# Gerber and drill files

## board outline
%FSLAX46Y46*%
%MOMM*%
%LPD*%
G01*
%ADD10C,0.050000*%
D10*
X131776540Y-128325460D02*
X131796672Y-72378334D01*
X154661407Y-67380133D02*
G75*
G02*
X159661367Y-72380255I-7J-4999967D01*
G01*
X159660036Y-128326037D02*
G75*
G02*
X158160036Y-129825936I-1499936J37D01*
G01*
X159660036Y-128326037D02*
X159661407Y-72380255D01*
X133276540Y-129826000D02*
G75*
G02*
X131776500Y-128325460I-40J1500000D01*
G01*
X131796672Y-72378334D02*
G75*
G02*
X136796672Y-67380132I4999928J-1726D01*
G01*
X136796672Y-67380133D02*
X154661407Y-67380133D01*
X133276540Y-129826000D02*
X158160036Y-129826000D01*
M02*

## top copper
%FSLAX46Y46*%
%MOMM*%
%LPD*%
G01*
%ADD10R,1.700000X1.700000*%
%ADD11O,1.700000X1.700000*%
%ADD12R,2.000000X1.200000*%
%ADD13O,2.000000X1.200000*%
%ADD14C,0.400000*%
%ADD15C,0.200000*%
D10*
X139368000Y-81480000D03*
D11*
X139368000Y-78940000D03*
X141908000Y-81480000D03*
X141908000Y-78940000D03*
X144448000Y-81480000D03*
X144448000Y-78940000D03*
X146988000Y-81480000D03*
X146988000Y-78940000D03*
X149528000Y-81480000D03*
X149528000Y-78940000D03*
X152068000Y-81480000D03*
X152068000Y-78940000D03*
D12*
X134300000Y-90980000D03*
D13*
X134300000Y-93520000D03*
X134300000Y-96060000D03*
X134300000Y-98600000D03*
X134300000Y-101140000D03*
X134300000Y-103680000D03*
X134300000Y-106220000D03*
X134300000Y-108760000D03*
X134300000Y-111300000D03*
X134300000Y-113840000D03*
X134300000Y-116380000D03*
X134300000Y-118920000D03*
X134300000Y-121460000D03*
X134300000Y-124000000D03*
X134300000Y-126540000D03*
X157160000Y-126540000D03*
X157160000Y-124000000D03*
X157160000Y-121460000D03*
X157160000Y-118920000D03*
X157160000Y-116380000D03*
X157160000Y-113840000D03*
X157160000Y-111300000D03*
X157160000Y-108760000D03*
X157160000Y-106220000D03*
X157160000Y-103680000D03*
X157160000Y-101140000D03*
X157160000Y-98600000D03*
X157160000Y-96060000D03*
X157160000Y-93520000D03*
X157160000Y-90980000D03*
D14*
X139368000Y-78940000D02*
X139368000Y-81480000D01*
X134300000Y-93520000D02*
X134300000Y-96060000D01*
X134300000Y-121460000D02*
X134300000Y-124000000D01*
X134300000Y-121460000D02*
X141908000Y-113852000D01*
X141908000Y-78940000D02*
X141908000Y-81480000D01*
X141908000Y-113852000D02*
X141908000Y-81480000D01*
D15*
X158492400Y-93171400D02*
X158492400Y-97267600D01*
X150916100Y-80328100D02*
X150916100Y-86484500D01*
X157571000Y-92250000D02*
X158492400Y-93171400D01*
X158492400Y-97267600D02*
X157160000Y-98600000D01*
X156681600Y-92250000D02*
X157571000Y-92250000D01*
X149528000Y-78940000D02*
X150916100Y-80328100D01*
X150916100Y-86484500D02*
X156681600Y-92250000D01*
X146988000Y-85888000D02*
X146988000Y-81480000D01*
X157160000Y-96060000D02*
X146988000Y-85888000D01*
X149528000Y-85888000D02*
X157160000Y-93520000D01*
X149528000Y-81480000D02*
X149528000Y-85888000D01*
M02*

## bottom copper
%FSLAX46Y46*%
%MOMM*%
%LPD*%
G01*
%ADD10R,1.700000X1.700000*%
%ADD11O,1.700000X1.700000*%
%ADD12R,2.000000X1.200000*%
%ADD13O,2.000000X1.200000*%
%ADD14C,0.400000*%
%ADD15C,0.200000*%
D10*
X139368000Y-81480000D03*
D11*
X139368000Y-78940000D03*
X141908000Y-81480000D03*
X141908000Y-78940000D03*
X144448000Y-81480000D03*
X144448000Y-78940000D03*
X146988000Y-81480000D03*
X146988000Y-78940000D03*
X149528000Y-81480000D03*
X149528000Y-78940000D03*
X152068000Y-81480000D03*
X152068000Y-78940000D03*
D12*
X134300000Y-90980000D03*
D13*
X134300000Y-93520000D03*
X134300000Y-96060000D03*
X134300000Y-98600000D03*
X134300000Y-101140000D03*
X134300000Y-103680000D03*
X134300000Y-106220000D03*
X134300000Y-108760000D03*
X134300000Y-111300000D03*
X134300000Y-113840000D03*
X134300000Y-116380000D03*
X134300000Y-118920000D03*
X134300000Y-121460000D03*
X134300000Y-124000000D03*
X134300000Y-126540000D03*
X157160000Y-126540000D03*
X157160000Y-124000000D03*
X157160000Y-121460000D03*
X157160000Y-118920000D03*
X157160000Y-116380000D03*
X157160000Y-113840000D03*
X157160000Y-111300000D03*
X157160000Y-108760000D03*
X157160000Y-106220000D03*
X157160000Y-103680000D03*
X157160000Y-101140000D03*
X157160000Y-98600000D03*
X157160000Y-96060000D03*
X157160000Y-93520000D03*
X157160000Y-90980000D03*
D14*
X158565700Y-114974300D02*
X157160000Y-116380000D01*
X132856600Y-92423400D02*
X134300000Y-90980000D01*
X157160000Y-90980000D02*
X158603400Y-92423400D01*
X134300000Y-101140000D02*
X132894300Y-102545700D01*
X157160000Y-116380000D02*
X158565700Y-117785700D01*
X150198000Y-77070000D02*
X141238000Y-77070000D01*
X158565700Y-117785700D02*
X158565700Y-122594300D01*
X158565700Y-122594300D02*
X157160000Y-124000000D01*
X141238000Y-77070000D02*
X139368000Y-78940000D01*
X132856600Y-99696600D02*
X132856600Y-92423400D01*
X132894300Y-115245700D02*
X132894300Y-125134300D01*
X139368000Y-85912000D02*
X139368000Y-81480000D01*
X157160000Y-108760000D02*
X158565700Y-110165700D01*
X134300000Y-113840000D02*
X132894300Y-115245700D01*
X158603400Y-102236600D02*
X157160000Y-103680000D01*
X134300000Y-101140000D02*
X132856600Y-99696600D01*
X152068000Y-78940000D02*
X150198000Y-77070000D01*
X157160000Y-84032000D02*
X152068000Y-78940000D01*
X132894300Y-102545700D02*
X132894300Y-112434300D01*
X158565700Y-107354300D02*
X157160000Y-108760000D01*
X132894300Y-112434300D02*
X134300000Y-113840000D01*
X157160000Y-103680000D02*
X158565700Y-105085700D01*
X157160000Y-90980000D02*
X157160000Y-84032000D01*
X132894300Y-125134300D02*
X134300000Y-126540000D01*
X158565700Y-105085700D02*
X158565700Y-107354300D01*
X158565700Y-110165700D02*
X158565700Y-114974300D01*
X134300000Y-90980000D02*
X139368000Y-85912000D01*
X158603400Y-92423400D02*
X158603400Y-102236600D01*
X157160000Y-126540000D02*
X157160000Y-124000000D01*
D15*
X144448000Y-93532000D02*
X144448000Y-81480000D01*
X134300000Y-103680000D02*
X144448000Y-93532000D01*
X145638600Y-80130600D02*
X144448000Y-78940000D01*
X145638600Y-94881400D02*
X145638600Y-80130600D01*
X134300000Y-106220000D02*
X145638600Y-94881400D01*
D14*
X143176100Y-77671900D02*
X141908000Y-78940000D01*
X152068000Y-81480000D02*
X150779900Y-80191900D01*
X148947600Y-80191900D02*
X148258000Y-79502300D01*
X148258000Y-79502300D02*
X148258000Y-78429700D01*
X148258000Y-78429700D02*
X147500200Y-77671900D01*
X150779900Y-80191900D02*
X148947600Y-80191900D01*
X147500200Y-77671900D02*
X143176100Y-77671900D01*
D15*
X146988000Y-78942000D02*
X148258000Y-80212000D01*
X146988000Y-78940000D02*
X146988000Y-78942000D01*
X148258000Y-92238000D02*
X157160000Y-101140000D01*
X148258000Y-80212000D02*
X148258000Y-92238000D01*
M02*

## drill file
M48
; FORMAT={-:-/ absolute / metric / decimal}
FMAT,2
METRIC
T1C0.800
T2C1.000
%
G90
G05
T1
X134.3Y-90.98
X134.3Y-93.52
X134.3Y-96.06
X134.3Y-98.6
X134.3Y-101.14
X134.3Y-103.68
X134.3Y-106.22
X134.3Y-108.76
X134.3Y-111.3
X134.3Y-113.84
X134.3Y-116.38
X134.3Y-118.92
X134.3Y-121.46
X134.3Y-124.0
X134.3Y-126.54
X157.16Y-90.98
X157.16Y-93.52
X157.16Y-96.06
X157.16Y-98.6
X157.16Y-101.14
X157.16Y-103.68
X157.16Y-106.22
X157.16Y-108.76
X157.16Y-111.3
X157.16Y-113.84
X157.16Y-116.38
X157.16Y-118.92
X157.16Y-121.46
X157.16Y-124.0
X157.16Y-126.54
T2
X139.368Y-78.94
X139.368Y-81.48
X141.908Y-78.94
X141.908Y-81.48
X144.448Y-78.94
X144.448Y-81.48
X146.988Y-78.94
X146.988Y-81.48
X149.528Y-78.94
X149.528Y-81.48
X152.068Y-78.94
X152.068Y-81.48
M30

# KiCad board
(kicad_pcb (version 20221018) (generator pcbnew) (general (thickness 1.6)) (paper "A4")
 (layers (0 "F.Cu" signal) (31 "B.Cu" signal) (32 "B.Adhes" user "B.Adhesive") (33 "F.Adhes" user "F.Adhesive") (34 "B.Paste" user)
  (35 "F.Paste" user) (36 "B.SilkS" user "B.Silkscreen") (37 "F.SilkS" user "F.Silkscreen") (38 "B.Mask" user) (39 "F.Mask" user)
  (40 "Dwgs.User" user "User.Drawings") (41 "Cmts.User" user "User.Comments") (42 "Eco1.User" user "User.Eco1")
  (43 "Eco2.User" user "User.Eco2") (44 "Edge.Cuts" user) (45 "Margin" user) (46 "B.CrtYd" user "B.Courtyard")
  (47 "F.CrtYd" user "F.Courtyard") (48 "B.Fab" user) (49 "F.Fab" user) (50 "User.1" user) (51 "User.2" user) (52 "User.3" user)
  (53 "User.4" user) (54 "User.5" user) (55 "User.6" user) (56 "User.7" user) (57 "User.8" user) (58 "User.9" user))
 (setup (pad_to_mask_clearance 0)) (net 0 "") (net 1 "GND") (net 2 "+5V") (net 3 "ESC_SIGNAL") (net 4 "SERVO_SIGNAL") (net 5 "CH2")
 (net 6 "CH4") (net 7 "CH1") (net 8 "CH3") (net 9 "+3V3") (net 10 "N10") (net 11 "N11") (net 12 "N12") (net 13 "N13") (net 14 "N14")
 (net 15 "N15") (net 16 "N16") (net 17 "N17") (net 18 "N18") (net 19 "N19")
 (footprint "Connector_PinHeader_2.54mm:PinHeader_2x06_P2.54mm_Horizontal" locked (layer "F.Cu") (at 139.368 81.48 90)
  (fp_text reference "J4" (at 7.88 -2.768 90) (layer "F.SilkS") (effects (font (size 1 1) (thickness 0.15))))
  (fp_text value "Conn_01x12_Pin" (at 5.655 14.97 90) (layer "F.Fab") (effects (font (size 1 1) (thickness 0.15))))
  (pad "1" thru_hole rect locked (at 0 0 90) (size 1.7 1.7) (drill 1) (layers "*.Cu" "*.Mask") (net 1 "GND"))
  (pad "2" thru_hole oval locked (at 2.54 0 90) (size 1.7 1.7) (drill 1) (layers "*.Cu" "*.Mask") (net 1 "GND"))
  (pad "3" thru_hole oval locked (at 0 2.54 90) (size 1.7 1.7) (drill 1) (layers "*.Cu" "*.Mask") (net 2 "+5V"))
  (pad "4" thru_hole oval locked (at 2.54 2.54 90) (size 1.7 1.7) (drill 1) (layers "*.Cu" "*.Mask") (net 2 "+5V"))
  (pad "5" thru_hole oval locked (at 0 5.08 90) (size 1.7 1.7) (drill 1) (layers "*.Cu" "*.Mask") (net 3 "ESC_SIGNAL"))
  (pad "6" thru_hole oval locked (at 2.54 5.08 90) (size 1.7 1.7) (drill 1) (layers "*.Cu" "*.Mask") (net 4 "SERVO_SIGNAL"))
  (pad "7" thru_hole oval locked (at 0 7.62 90) (size 1.7 1.7) (drill 1) (layers "*.Cu" "*.Mask") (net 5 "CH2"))
  (pad "8" thru_hole oval locked (at 2.54 7.62 90) (size 1.7 1.7) (drill 1) (layers "*.Cu" "*.Mask") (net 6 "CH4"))
  (pad "9" thru_hole oval locked (at 0 10.16 90) (size 1.7 1.7) (drill 1) (layers "*.Cu" "*.Mask") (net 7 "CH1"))
  (pad "10" thru_hole oval locked (at 2.54 10.16 90) (size 1.7 1.7) (drill 1) (layers "*.Cu" "*.Mask") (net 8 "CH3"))
  (pad "11" thru_hole oval locked (at 0 12.7 90) (size 1.7 1.7) (drill 1) (layers "*.Cu" "*.Mask") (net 2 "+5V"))
  (pad "12" thru_hole oval locked (at 2.54 12.7 90) (size 1.7 1.7) (drill 1) (layers "*.Cu" "*.Mask") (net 1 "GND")))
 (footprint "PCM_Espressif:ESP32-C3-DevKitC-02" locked (layer "F.Cu") (at 134.3 90.98)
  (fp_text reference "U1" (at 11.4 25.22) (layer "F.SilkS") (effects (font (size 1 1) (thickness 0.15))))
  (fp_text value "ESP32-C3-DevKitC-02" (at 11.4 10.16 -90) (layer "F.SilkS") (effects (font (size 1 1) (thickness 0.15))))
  (pad "1" thru_hole rect locked (at 0 0 270) (size 1.2 2) (drill 0.8) (layers "*.Cu" "*.Mask") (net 1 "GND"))
  (pad "2" thru_hole oval locked (at 0 2.54 270) (size 1.2 2) (drill 0.8) (layers "*.Cu" "*.Mask") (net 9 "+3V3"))
  (pad "3" thru_hole oval locked (at 0 5.08 270) (size 1.2 2) (drill 0.8) (layers "*.Cu" "*.Mask") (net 9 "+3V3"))
  (pad "4" thru_hole oval locked (at 0 7.62 270) (size 1.2 2) (drill 0.8) (layers "*.Cu" "*.Mask") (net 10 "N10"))
  (pad "5" thru_hole oval locked (at 0 10.16 270) (size 1.2 2) (drill 0.8) (layers "*.Cu" "*.Mask") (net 1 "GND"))
  (pad "6" thru_hole oval locked (at 0 12.7 270) (size 1.2 2) (drill 0.8) (layers "*.Cu" "*.Mask") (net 3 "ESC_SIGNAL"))
  (pad "7" thru_hole oval locked (at 0 15.24 270) (size 1.2 2) (drill 0.8) (layers "*.Cu" "*.Mask") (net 4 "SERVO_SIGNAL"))
  (pad "8" thru_hole oval locked (at 0 17.78 270) (size 1.2 2) (drill 0.8) (layers "*.Cu" "*.Mask") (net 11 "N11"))
  (pad "9" thru_hole oval locked (at 0 20.32 270) (size 1.2 2) (drill 0.8) (layers "*.Cu" "*.Mask") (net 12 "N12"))
  (pad "10" thru_hole oval locked (at 0 22.86 270) (size 1.2 2) (drill 0.8) (layers "*.Cu" "*.Mask") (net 1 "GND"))
  (pad "11" thru_hole oval locked (at 0 25.4 270) (size 1.2 2) (drill 0.8) (layers "*.Cu" "*.Mask") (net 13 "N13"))
  (pad "12" thru_hole oval locked (at 0 27.94 270) (size 1.2 2) (drill 0.8) (layers "*.Cu" "*.Mask") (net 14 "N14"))
  (pad "13" thru_hole oval locked (at 0 30.48 270) (size 1.2 2) (drill 0.8) (layers "*.Cu" "*.Mask") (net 2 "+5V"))
  (pad "14" thru_hole oval locked (at 0 33.02 270) (size 1.2 2) (drill 0.8) (layers "*.Cu" "*.Mask") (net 2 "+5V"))
  (pad "15" thru_hole oval locked (at 0 35.56 270) (size 1.2 2) (drill 0.8) (layers "*.Cu" "*.Mask") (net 1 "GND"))
  (pad "16" thru_hole oval locked (at 22.86 35.56 270) (size 1.2 2) (drill 0.8) (layers "*.Cu" "*.Mask") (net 1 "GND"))
  (pad "17" thru_hole oval locked (at 22.86 33.02 270) (size 1.2 2) (drill 0.8) (layers "*.Cu" "*.Mask") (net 1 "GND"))
  (pad "18" thru_hole oval locked (at 22.86 30.48 270) (size 1.2 2) (drill 0.8) (layers "*.Cu" "*.Mask") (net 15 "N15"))
  (pad "19" thru_hole oval locked (at 22.86 27.94 270) (size 1.2 2) (drill 0.8) (layers "*.Cu" "*.Mask") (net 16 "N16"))
  (pad "20" thru_hole oval locked (at 22.86 25.4 270) (size 1.2 2) (drill 0.8) (layers "*.Cu" "*.Mask") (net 1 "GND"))
  (pad "21" thru_hole oval locked (at 22.86 22.86 270) (size 1.2 2) (drill 0.8) (layers "*.Cu" "*.Mask") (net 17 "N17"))
  (pad "22" thru_hole oval locked (at 22.86 20.32 270) (size 1.2 2) (drill 0.8) (layers "*.Cu" "*.Mask") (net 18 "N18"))
  (pad "23" thru_hole oval locked (at 22.86 17.78 270) (size 1.2 2) (drill 0.8) (layers "*.Cu" "*.Mask") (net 1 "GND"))
  (pad "24" thru_hole oval locked (at 22.86 15.24 270) (size 1.2 2) (drill 0.8) (layers "*.Cu" "*.Mask") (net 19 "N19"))
  (pad "25" thru_hole oval locked (at 22.86 12.7 270) (size 1.2 2) (drill 0.8) (layers "*.Cu" "*.Mask") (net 1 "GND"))
  (pad "26" thru_hole oval locked (at 22.86 10.16 270) (size 1.2 2) (drill 0.8) (layers "*.Cu" "*.Mask") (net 6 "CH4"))
  (pad "27" thru_hole oval locked (at 22.86 7.62 270) (size 1.2 2) (drill 0.8) (layers "*.Cu" "*.Mask") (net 8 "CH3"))
  (pad "28" thru_hole oval locked (at 22.86 5.08 270) (size 1.2 2) (drill 0.8) (layers "*.Cu" "*.Mask") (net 5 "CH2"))
  (pad "29" thru_hole oval locked (at 22.86 2.54 270) (size 1.2 2) (drill 0.8) (layers "*.Cu" "*.Mask") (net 7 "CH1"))
  (pad "30" thru_hole oval locked (at 22.86 0 270) (size 1.2 2) (drill 0.8) (layers "*.Cu" "*.Mask") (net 1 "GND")))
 (gr_line (start 131.77654 128.32546) (end 131.796672 72.378334) (stroke (width 0.05) (type default)) (layer "Edge.Cuts"))
 (gr_arc (start 154.661407 67.380133) (mid 158.196984 68.844642) (end 159.661407 72.380255) (stroke (width 0.05) (type default))
  (layer "Edge.Cuts"))
 (gr_arc (start 159.660036 128.326037) (mid 159.220685 129.386686) (end 158.160036 129.826) (stroke (width 0.05) (type default))
  (layer "Edge.Cuts"))
 (gr_line (start 159.660036 128.326037) (end 159.661407 72.380255) (stroke (width 0.05) (type default)) (layer "Edge.Cuts"))
 (gr_arc (start 133.27654 129.826) (mid 132.215689 129.386469) (end 131.77654 128.32546) (stroke (width 0.05) (type default))
  (layer "Edge.Cuts"))
 (gr_arc (start 131.796672 72.378334) (mid 133.261761 68.843932) (end 136.796672 67.380133) (stroke (width 0.05) (type default))
  (layer "Edge.Cuts"))
 (gr_line (start 136.796672 67.380133) (end 154.661407 67.380133) (stroke (width 0.05) (type default)) (layer "Edge.Cuts"))
 (gr_line (start 133.27654 129.826) (end 158.160036 129.826) (stroke (width 0.05) (type default)) (layer "Edge.Cuts"))
 (segment (start 139.368 78.94) (end 139.368 81.48) (width 0.4) (layer "F.Cu") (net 1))
 (segment (start 158.5657 114.9743) (end 157.16 116.38) (width 0.4) (layer "B.Cu") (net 1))
 (segment (start 132.8566 92.4234) (end 134.3 90.98) (width 0.4) (layer "B.Cu") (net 1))
 (segment (start 157.16 90.98) (end 158.6034 92.4234) (width 0.4) (layer "B.Cu") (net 1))
 (segment (start 134.3 101.14) (end 132.8943 102.5457) (width 0.4) (layer "B.Cu") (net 1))
 (segment (start 157.16 116.38) (end 158.5657 117.7857) (width 0.4) (layer "B.Cu") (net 1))
 (segment (start 150.198 77.07) (end 141.238 77.07) (width 0.4) (layer "B.Cu") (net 1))
 (segment (start 158.5657 117.7857) (end 158.5657 122.5943) (width 0.4) (layer "B.Cu") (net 1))
 (segment (start 158.5657 122.5943) (end 157.16 124) (width 0.4) (layer "B.Cu") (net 1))
 (segment (start 141.238 77.07) (end 139.368 78.94) (width 0.4) (layer "B.Cu") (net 1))
 (segment (start 132.8566 99.6966) (end 132.8566 92.4234) (width 0.4) (layer "B.Cu") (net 1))
 (segment (start 132.8943 115.2457) (end 132.8943 125.1343) (width 0.4) (layer "B.Cu") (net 1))
 (segment (start 139.368 85.912) (end 139.368 81.48) (width 0.4) (layer "B.Cu") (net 1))
 (segment (start 157.16 108.76) (end 158.5657 110.1657) (width 0.4) (layer "B.Cu") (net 1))
 (segment (start 134.3 113.84) (end 132.8943 115.2457) (width 0.4) (layer "B.Cu") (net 1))
 (segment (start 158.6034 102.2366) (end 157.16 103.68) (width 0.4) (layer "B.Cu") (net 1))
 (segment (start 134.3 101.14) (end 132.8566 99.6966) (width 0.4) (layer "B.Cu") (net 1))
 (segment (start 152.068 78.94) (end 150.198 77.07) (width 0.4) (layer "B.Cu") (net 1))
 (segment (start 157.16 84.032) (end 152.068 78.94) (width 0.4) (layer "B.Cu") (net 1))
 (segment (start 132.8943 102.5457) (end 132.8943 112.4343) (width 0.4) (layer "B.Cu") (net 1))
 (segment (start 158.5657 107.3543) (end 157.16 108.76) (width 0.4) (layer "B.Cu") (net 1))
 (segment (start 132.8943 112.4343) (end 134.3 113.84) (width 0.4) (layer "B.Cu") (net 1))
 (segment (start 157.16 103.68) (end 158.5657 105.0857) (width 0.4) (layer "B.Cu") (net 1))
 (segment (start 157.16 90.98) (end 157.16 84.032) (width 0.4) (layer "B.Cu") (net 1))
 (segment (start 132.8943 125.1343) (end 134.3 126.54) (width 0.4) (layer "B.Cu") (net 1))
 (segment (start 158.5657 105.0857) (end 158.5657 107.3543) (width 0.4) (layer "B.Cu") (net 1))
 (segment (start 158.5657 110.1657) (end 158.5657 114.9743) (width 0.4) (layer "B.Cu") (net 1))
 (segment (start 134.3 90.98) (end 139.368 85.912) (width 0.4) (layer "B.Cu") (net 1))
 (segment (start 158.6034 92.4234) (end 158.6034 102.2366) (width 0.4) (layer "B.Cu") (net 1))
 (segment (start 157.16 126.54) (end 157.16 124) (width 0.4) (layer "B.Cu") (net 1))
 (segment (start 134.3 93.52) (end 134.3 96.06) (width 0.4) (layer "F.Cu") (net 9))
 (segment (start 144.448 93.532) (end 144.448 81.48) (width 0.2) (layer "B.Cu") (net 3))
 (segment (start 134.3 103.68) (end 144.448 93.532) (width 0.2) (layer "B.Cu") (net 3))
 (segment (start 145.6386 80.1306) (end 144.448 78.94) (width 0.2) (layer "B.Cu") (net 4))
 (segment (start 145.6386 94.8814) (end 145.6386 80.1306) (width 0.2) (layer "B.Cu") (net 4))
 (segment (start 134.3 106.22) (end 145.6386 94.8814) (width 0.2) (layer "B.Cu") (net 4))
 (segment (start 134.3 121.46) (end 134.3 124) (width 0.4) (layer "F.Cu") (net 2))
 (segment (start 134.3 121.46) (end 141.908 113.852) (width 0.4) (layer "F.Cu") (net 2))
 (segment (start 141.908 78.94) (end 141.908 81.48) (width 0.4) (layer "F.Cu") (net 2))
 (segment (start 141.908 113.852) (end 141.908 81.48) (width 0.4) (layer "F.Cu") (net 2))
 (segment (start 143.1761 77.6719) (end 141.908 78.94) (width 0.4) (layer "B.Cu") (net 2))
 (segment (start 152.068 81.48) (end 150.7799 80.1919) (width 0.4) (layer "B.Cu") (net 2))
 (segment (start 148.9476 80.1919) (end 148.258 79.5023) (width 0.4) (layer "B.Cu") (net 2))
 (segment (start 148.258 79.5023) (end 148.258 78.4297) (width 0.4) (layer "B.Cu") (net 2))
 (segment (start 148.258 78.4297) (end 147.5002 77.6719) (width 0.4) (layer "B.Cu") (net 2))
 (segment (start 150.7799 80.1919) (end 148.9476 80.1919) (width 0.4) (layer "B.Cu") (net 2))
 (segment (start 147.5002 77.6719) (end 143.1761 77.6719) (width 0.4) (layer "B.Cu") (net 2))
 (segment (start 146.988 78.942) (end 148.258 80.212) (width 0.2) (layer "B.Cu") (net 6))
 (segment (start 146.988 78.94) (end 146.988 78.942) (width 0.2) (layer "B.Cu") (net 6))
 (segment (start 148.258 92.238) (end 157.16 101.14) (width 0.2) (layer "B.Cu") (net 6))
 (segment (start 148.258 80.212) (end 148.258 92.238) (width 0.2) (layer "B.Cu") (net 6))
 (segment (start 158.4924 93.1714) (end 158.4924 97.2676) (width 0.2) (layer "F.Cu") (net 8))
 (segment (start 150.9161 80.3281) (end 150.9161 86.4845) (width 0.2) (layer "F.Cu") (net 8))
 (segment (start 157.571 92.25) (end 158.4924 93.1714) (width 0.2) (layer "F.Cu") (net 8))
 (segment (start 158.4924 97.2676) (end 157.16 98.6) (width 0.2) (layer "F.Cu") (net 8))
 (segment (start 156.6816 92.25) (end 157.571 92.25) (width 0.2) (layer "F.Cu") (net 8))
 (segment (start 149.528 78.94) (end 150.9161 80.3281) (width 0.2) (layer "F.Cu") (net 8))
 (segment (start 150.9161 86.4845) (end 156.6816 92.25) (width 0.2) (layer "F.Cu") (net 8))
 (segment (start 146.988 85.888) (end 146.988 81.48) (width 0.2) (layer "F.Cu") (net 5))
 (segment (start 157.16 96.06) (end 146.988 85.888) (width 0.2) (layer "F.Cu") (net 5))
 (segment (start 149.528 85.888) (end 157.16 93.52) (width 0.2) (layer "F.Cu") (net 7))
 (segment (start 149.528 81.48) (end 149.528 85.888) (width 0.2) (layer "F.Cu") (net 7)))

